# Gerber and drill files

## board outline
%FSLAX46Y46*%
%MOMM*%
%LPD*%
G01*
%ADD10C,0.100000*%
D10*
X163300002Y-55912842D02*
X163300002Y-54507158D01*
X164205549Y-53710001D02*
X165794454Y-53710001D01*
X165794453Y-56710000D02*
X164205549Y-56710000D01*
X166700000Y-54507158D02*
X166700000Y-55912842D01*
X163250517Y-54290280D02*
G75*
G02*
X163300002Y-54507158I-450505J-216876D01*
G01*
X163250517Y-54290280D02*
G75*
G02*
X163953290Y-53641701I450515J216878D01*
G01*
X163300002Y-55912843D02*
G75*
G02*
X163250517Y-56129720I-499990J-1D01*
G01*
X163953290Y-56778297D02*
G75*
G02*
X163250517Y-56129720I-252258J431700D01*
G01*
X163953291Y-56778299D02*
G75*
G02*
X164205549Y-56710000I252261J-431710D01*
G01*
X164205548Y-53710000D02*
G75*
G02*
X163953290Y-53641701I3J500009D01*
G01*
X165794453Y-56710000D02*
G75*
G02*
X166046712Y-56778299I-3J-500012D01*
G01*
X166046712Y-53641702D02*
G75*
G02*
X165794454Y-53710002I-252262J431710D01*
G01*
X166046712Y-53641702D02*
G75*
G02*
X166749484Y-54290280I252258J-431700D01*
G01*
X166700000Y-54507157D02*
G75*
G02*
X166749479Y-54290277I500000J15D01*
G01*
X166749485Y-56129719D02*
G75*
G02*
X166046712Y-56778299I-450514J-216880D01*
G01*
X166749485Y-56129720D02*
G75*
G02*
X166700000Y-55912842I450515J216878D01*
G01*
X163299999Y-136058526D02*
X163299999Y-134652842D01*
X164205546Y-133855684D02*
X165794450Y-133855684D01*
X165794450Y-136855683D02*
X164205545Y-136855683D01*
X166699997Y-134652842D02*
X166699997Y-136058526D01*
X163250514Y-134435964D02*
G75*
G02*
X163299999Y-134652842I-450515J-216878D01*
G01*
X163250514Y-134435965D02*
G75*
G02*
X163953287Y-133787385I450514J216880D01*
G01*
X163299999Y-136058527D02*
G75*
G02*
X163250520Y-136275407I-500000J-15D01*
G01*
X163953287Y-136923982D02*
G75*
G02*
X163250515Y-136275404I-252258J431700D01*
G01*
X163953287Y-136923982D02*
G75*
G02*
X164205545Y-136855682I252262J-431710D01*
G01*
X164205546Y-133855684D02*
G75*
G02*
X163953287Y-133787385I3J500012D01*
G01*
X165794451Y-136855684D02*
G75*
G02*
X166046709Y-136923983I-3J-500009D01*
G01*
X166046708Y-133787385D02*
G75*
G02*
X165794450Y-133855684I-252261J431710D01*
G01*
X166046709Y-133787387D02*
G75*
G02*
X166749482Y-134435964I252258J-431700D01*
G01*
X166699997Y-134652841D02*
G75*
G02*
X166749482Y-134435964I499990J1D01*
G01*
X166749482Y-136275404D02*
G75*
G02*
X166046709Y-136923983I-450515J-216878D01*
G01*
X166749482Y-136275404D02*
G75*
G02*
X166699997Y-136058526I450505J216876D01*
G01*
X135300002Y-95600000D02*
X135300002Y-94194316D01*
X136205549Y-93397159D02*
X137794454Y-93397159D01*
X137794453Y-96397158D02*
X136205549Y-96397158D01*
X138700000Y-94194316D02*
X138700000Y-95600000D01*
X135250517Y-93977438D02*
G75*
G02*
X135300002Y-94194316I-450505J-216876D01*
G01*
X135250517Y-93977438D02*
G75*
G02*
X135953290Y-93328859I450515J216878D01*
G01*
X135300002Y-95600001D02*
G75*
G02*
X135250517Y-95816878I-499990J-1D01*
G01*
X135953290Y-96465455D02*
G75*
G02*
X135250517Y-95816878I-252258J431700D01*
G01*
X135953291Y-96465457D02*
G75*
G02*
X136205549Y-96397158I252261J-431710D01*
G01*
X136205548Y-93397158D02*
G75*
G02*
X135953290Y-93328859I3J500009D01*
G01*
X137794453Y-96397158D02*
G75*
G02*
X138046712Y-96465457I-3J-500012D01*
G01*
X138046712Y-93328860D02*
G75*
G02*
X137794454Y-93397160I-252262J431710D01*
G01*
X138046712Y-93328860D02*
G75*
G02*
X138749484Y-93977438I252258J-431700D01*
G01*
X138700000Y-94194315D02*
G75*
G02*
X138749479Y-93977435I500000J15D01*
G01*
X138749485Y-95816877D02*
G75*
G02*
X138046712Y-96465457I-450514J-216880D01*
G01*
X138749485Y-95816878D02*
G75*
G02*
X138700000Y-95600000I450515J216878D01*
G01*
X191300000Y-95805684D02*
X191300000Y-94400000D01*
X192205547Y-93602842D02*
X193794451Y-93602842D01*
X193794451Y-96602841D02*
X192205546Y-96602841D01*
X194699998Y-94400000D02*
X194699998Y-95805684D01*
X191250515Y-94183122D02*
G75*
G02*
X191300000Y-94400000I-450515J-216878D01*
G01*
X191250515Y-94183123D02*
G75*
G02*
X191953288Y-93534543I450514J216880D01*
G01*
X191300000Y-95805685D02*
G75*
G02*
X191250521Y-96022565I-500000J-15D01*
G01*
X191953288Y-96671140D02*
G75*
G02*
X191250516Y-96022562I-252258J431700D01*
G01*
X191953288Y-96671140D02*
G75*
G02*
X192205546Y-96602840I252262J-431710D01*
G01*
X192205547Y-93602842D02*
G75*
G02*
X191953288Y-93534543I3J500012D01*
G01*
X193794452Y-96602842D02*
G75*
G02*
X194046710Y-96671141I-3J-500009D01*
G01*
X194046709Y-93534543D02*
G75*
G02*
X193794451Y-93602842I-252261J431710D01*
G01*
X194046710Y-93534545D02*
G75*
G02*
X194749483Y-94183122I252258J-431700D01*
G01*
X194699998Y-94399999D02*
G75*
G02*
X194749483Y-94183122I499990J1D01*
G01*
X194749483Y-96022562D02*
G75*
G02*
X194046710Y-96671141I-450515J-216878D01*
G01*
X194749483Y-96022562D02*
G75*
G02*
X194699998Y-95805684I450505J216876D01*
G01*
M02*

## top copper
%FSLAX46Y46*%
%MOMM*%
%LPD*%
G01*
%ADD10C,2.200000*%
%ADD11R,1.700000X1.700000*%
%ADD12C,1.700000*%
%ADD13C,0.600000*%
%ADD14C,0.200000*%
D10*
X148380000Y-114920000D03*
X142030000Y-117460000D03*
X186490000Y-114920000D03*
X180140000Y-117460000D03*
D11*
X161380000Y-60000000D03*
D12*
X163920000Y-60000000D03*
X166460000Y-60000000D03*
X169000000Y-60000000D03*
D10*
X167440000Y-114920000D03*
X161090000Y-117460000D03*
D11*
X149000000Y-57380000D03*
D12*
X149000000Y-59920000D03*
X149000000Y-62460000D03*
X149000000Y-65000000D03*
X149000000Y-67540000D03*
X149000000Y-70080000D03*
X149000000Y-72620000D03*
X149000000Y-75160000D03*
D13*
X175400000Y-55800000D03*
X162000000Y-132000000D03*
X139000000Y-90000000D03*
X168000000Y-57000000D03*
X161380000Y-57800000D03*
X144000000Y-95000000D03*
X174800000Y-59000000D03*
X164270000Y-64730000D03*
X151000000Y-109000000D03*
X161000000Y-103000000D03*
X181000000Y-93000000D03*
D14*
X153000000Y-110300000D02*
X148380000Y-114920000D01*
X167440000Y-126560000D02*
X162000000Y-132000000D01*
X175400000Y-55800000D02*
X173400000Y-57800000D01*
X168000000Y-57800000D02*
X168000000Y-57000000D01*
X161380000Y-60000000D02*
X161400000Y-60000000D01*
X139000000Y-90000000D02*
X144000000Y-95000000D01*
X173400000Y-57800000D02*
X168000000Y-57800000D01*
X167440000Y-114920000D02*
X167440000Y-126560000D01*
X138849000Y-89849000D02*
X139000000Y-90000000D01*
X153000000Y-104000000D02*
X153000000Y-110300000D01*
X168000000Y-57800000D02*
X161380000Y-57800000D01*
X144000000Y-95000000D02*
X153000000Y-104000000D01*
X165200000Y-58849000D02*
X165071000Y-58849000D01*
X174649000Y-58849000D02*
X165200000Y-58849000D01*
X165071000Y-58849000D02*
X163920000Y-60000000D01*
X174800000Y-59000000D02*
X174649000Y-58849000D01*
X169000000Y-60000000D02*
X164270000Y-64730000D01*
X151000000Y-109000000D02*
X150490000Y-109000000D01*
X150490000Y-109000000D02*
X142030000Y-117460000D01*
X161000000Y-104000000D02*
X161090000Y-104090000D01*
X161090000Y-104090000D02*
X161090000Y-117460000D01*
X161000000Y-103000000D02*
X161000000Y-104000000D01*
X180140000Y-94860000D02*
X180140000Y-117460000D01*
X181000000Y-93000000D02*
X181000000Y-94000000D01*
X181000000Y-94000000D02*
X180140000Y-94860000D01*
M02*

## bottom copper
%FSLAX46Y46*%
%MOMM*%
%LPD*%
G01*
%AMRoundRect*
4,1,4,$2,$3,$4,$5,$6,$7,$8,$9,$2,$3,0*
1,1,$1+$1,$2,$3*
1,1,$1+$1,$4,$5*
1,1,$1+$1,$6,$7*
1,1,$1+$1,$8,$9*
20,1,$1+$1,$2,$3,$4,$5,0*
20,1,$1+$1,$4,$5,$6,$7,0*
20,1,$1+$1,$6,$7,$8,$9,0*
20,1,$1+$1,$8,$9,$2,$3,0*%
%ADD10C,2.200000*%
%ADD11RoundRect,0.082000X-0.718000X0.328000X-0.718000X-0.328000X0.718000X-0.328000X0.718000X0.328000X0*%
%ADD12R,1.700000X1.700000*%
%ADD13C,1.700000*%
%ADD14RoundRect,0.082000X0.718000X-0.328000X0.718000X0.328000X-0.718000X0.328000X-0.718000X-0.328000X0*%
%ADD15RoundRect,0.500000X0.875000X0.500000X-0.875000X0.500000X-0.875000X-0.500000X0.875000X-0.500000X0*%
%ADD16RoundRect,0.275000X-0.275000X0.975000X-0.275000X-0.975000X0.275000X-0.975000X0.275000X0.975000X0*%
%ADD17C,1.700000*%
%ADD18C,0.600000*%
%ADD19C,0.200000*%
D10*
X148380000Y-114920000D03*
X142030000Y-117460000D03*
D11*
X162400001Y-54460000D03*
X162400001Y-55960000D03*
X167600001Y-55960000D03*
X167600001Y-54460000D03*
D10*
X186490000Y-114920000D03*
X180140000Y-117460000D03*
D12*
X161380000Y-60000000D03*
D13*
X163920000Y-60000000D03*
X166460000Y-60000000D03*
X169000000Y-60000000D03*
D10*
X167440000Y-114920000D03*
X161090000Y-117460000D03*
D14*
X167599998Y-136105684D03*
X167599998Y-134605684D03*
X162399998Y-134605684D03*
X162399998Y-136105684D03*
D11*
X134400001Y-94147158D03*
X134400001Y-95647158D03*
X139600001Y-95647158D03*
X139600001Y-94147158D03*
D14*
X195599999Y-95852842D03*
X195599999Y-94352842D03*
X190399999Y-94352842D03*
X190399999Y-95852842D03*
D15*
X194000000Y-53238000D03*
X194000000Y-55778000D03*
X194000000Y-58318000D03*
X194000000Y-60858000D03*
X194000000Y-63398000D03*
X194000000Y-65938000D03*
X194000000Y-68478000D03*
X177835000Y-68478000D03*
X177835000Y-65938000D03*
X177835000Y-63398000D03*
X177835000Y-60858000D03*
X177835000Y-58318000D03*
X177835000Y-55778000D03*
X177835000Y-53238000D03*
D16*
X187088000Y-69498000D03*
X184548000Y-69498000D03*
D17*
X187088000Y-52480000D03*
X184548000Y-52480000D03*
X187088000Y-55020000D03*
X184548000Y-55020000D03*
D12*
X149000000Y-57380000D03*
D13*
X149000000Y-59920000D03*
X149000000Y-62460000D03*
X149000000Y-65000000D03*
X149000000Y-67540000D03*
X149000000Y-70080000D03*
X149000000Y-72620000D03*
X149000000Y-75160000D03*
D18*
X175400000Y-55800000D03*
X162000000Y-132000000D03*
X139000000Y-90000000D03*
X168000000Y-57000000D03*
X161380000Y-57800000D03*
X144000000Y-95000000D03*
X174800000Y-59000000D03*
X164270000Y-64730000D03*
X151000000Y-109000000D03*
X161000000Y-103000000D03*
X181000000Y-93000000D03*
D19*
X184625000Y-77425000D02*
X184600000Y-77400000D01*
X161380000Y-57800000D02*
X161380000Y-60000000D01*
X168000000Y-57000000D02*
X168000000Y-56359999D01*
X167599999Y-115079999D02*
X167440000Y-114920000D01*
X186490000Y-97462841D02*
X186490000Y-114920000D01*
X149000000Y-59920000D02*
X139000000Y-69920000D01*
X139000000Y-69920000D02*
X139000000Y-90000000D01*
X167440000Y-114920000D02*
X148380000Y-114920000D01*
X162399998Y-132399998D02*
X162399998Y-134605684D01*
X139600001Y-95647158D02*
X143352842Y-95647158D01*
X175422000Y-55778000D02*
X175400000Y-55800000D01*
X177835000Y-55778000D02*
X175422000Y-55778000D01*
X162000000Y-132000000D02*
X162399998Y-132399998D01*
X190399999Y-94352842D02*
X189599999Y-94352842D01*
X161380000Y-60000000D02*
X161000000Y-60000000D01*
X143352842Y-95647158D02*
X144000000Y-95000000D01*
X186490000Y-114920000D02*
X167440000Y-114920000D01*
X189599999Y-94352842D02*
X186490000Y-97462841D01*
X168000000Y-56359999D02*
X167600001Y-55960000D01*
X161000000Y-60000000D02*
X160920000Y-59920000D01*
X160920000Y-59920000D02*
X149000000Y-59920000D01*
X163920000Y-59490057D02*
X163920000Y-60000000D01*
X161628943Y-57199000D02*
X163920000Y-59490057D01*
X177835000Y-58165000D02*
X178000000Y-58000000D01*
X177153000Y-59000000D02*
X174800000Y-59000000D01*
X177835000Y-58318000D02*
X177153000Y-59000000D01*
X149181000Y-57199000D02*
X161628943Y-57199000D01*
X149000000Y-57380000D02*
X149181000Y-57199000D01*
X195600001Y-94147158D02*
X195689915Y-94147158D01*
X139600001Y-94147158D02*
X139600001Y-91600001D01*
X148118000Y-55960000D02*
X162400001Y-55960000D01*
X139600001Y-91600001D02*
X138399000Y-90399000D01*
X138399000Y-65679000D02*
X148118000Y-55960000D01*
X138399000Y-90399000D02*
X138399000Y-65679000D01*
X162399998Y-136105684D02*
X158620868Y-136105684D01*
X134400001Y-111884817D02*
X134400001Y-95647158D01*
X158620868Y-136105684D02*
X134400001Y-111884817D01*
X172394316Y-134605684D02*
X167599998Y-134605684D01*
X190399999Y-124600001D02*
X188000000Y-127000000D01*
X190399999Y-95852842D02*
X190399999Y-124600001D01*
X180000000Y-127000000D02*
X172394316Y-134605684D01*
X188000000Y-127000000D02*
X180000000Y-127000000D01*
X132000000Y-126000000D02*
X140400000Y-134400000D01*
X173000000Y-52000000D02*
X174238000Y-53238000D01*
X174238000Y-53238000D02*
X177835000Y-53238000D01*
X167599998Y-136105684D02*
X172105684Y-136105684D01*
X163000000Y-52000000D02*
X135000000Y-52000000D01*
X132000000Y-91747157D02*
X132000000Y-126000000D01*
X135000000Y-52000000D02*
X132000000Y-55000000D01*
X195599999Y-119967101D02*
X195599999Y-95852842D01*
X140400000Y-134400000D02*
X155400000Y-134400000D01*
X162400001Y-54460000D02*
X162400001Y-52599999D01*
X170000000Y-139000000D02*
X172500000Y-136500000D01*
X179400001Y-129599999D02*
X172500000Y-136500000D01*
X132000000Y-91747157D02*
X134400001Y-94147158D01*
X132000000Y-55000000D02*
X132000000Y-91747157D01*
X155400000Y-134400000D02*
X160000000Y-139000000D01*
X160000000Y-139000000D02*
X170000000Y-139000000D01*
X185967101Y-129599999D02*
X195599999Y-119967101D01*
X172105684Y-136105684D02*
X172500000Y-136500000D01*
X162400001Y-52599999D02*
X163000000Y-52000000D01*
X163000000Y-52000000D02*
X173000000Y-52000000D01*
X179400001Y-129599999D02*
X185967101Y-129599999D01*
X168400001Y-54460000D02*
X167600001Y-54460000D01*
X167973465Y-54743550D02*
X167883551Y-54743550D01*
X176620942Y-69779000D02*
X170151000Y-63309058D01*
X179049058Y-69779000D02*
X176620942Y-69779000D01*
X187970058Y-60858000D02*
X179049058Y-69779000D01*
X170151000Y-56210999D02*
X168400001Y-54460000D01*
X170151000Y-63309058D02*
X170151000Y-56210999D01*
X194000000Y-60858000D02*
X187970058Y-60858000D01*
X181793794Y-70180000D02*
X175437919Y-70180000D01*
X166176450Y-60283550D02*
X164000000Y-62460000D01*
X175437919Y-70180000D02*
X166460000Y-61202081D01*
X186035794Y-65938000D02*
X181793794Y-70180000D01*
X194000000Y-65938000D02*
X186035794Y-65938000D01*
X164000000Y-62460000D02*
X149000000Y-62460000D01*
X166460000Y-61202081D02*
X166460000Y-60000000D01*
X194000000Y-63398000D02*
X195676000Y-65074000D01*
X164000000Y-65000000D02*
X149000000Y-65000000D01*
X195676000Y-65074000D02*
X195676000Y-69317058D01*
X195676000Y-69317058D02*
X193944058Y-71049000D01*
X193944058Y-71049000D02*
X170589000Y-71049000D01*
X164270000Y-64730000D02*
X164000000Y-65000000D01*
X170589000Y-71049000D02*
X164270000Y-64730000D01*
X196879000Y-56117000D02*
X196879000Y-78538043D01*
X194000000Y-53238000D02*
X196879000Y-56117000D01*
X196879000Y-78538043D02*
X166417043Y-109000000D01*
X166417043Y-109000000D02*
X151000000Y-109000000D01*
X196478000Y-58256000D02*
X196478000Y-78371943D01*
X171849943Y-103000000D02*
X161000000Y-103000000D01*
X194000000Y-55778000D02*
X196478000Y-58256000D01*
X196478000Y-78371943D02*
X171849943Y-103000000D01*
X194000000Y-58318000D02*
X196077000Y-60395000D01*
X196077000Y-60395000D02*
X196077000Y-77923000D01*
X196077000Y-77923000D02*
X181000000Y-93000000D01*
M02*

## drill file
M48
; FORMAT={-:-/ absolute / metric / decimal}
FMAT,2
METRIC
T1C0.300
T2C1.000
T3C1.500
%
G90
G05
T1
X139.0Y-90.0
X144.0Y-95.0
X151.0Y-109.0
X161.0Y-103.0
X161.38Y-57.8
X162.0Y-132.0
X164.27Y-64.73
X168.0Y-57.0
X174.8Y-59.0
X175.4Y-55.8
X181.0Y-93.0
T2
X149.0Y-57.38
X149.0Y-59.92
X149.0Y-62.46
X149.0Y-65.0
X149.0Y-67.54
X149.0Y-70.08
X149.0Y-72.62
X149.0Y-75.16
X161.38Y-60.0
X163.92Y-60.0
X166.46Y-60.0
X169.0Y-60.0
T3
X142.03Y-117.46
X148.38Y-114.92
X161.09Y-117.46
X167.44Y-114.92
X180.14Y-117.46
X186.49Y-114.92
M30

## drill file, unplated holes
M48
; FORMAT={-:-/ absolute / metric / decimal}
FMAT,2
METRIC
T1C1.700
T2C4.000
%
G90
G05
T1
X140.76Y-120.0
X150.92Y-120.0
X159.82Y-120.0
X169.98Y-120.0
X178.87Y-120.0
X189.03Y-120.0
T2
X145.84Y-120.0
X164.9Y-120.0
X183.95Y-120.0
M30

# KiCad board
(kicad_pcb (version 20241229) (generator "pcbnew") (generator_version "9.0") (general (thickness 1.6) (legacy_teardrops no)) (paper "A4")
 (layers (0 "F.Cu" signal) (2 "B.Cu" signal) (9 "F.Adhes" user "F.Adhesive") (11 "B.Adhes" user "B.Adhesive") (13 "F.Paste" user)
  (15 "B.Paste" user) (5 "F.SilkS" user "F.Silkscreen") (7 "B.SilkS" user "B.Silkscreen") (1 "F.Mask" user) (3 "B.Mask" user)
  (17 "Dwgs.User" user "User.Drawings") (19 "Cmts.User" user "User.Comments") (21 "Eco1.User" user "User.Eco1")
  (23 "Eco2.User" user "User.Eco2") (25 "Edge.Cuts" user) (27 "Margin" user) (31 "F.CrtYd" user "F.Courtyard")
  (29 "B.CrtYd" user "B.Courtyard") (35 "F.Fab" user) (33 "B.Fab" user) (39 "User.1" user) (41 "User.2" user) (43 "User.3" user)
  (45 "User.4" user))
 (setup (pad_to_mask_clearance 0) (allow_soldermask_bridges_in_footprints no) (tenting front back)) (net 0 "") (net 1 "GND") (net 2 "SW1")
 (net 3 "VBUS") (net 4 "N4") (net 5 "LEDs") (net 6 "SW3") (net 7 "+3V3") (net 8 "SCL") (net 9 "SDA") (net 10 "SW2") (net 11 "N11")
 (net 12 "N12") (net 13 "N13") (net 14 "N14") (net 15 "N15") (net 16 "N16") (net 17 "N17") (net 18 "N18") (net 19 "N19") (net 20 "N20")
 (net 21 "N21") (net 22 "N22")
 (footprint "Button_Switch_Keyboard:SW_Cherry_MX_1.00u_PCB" (layer "F.Cu") (at 148.38 114.92)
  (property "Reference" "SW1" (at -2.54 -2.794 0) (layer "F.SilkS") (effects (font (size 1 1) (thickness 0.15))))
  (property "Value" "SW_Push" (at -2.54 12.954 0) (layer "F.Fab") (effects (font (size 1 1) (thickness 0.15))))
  (pad "" np_thru_hole circle (at -7.62 5.08) (size 1.7 1.7) (drill 1.7) (layers "*.Cu" "*.Mask"))
  (pad "" np_thru_hole circle (at -2.54 5.08) (size 4 4) (drill 4) (layers "*.Cu" "*.Mask"))
  (pad "" np_thru_hole circle (at 2.54 5.08) (size 1.7 1.7) (drill 1.7) (layers "*.Cu" "*.Mask"))
  (pad "1" thru_hole circle (at 0 0) (size 2.2 2.2) (drill 1.5) (layers "*.Cu" "*.Mask") (remove_unused_layers no) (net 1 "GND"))
  (pad "2" thru_hole circle (at -6.35 2.54) (size 2.2 2.2) (drill 1.5) (layers "*.Cu" "*.Mask") (remove_unused_layers no) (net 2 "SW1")))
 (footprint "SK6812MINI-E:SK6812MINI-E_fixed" (layer "F.Cu") (at 165 55.312842)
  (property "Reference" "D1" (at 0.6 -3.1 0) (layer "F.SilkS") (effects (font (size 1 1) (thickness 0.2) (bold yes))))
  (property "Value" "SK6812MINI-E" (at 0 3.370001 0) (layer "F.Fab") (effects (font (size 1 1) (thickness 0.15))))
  (fp_line (start -1.699998 0.6) (end -1.699998 -0.805684) (stroke (width 0.1) (type solid)) (layer "Edge.Cuts"))
  (fp_line (start -0.794451 -1.602841) (end 0.794454 -1.602841) (stroke (width 0.1) (type solid)) (layer "Edge.Cuts"))
  (fp_line (start 0.794453 1.397158) (end -0.794451 1.397158) (stroke (width 0.1) (type solid)) (layer "Edge.Cuts"))
  (fp_line (start 1.7 -0.805684) (end 1.7 0.6) (stroke (width 0.1) (type solid)) (layer "Edge.Cuts"))
  (fp_arc (start -1.749483 -1.022562) (mid -1.712526 -0.91691) (end -1.699998 -0.805684) (stroke (width 0.1) (type solid))
   (layer "Edge.Cuts"))
  (fp_arc (start -1.749483 -1.022562) (mid -1.63807 -1.606877) (end -1.04671 -1.671141) (stroke (width 0.1) (type solid))
   (layer "Edge.Cuts"))
  (fp_arc (start -1.699998 0.600001) (mid -1.712526 0.711226) (end -1.749483 0.816878) (stroke (width 0.1) (type solid)) (layer "Edge.Cuts"))
  (fp_arc (start -1.04671 1.465455) (mid -1.638069 1.401192) (end -1.749483 0.816878) (stroke (width 0.1) (type solid)) (layer "Edge.Cuts"))
  (fp_arc (start -1.046709 1.465457) (mid -0.925121 1.414535) (end -0.794451 1.397158) (stroke (width 0.1) (type solid)) (layer "Edge.Cuts"))
  (fp_arc (start -0.794452 -1.602842) (mid -0.925122 -1.620219) (end -1.04671 -1.671141) (stroke (width 0.1) (type solid))
   (layer "Edge.Cuts"))
  (fp_arc (start 0.794453 1.397158) (mid 0.925124 1.414535) (end 1.046712 1.465457) (stroke (width 0.1) (type solid)) (layer "Edge.Cuts"))
  (fp_arc (start 1.046712 -1.67114) (mid 0.925124 -1.620218) (end 0.794454 -1.602841) (stroke (width 0.1) (type solid)) (layer "Edge.Cuts"))
  (fp_arc (start 1.046712 -1.67114) (mid 1.638072 -1.606876) (end 1.749485 -1.022562) (stroke (width 0.1) (type solid)) (layer "Edge.Cuts"))
  (fp_arc (start 1.7 -0.805685) (mid 1.712528 -0.91691) (end 1.749485 -1.022562) (stroke (width 0.1) (type solid)) (layer "Edge.Cuts"))
  (fp_arc (start 1.749485 0.816877) (mid 1.638073 1.401193) (end 1.046712 1.465457) (stroke (width 0.1) (type solid)) (layer "Edge.Cuts"))
  (fp_arc (start 1.749485 0.816878) (mid 1.712528 0.711226) (end 1.7 0.6) (stroke (width 0.1) (type solid)) (layer "Edge.Cuts"))
  (pad "1" smd roundrect (at -2.599999 -0.852842 270) (size 0.82 1.6) (layers "B.Cu" "B.Mask" "B.Paste") (roundrect_rratio 0.1)
   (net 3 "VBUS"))
  (pad "2" smd roundrect (at -2.599999 0.647158 270) (size 0.82 1.6) (layers "B.Cu" "B.Mask" "B.Paste") (roundrect_rratio 0.1) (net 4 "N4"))
  (pad "3" smd roundrect (at 2.600001 0.647158 270) (size 0.82 1.6) (layers "B.Cu" "B.Mask" "B.Paste") (roundrect_rratio 0.1) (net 1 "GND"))
  (pad "4" smd roundrect (at 2.600001 -0.852842 270) (size 0.82 1.6) (layers "B.Cu" "B.Mask" "B.Paste") (roundrect_rratio 0.1)
   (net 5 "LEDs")))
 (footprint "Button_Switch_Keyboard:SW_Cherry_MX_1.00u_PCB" (layer "F.Cu") (at 186.49 114.92)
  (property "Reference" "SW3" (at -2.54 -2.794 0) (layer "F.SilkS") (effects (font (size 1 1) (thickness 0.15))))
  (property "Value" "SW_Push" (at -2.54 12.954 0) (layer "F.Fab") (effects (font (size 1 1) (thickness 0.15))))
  (pad "" np_thru_hole circle (at -7.62 5.08) (size 1.7 1.7) (drill 1.7) (layers "*.Cu" "*.Mask"))
  (pad "" np_thru_hole circle (at -2.54 5.08) (size 4 4) (drill 4) (layers "*.Cu" "*.Mask"))
  (pad "" np_thru_hole circle (at 2.54 5.08) (size 1.7 1.7) (drill 1.7) (layers "*.Cu" "*.Mask"))
  (pad "1" thru_hole circle (at 0 0) (size 2.2 2.2) (drill 1.5) (layers "*.Cu" "*.Mask") (remove_unused_layers no) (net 1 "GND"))
  (pad "2" thru_hole circle (at -6.35 2.54) (size 2.2 2.2) (drill 1.5) (layers "*.Cu" "*.Mask") (remove_unused_layers no) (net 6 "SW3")))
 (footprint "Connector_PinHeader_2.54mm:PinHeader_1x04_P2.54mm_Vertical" (layer "F.Cu") (at 161.38 60 90)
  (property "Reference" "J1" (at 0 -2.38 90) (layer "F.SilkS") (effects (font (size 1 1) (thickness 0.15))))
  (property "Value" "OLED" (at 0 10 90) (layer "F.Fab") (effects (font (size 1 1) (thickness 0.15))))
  (pad "1" thru_hole rect (at 0 0 90) (size 1.7 1.7) (drill 1) (layers "*.Cu" "*.Mask") (remove_unused_layers no) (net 1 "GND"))
  (pad "2" thru_hole circle (at 0 2.54 90) (size 1.7 1.7) (drill 1) (layers "*.Cu" "*.Mask") (remove_unused_layers no) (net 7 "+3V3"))
  (pad "3" thru_hole circle (at 0 5.08 90) (size 1.7 1.7) (drill 1) (layers "*.Cu" "*.Mask") (remove_unused_layers no) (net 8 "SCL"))
  (pad "4" thru_hole circle (at 0 7.62 90) (size 1.7 1.7) (drill 1) (layers "*.Cu" "*.Mask") (remove_unused_layers no) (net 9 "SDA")))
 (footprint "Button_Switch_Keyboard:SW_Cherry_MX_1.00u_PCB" (layer "F.Cu") (at 167.44 114.92)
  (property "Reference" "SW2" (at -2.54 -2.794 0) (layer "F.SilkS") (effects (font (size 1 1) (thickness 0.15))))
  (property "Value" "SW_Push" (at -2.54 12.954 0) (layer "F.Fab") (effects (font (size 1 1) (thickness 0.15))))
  (pad "" np_thru_hole circle (at -7.62 5.08) (size 1.7 1.7) (drill 1.7) (layers "*.Cu" "*.Mask"))
  (pad "" np_thru_hole circle (at -2.54 5.08) (size 4 4) (drill 4) (layers "*.Cu" "*.Mask"))
  (pad "" np_thru_hole circle (at 2.54 5.08) (size 1.7 1.7) (drill 1.7) (layers "*.Cu" "*.Mask"))
  (pad "1" thru_hole circle (at 0 0) (size 2.2 2.2) (drill 1.5) (layers "*.Cu" "*.Mask") (remove_unused_layers no) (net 1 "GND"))
  (pad "2" thru_hole circle (at -6.35 2.54) (size 2.2 2.2) (drill 1.5) (layers "*.Cu" "*.Mask") (remove_unused_layers no) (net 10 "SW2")))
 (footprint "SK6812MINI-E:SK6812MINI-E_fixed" (layer "F.Cu") (at 164.999999 135.252842 180)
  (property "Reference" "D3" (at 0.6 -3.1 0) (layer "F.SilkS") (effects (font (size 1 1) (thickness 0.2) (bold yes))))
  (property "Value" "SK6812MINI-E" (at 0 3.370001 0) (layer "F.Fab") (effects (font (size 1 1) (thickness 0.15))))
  (fp_line (start 1.7 -0.805684) (end 1.7 0.6) (stroke (width 0.1) (type solid)) (layer "Edge.Cuts"))
  (fp_line (start 0.794453 1.397158) (end -0.794451 1.397158) (stroke (width 0.1) (type solid)) (layer "Edge.Cuts"))
  (fp_line (start -0.794451 -1.602841) (end 0.794454 -1.602841) (stroke (width 0.1) (type solid)) (layer "Edge.Cuts"))
  (fp_line (start -1.699998 0.6) (end -1.699998 -0.805684) (stroke (width 0.1) (type solid)) (layer "Edge.Cuts"))
  (fp_arc (start 1.749485 0.816878) (mid 1.712528 0.711226) (end 1.7 0.6) (stroke (width 0.1) (type solid)) (layer "Edge.Cuts"))
  (fp_arc (start 1.749485 0.816877) (mid 1.638073 1.401193) (end 1.046712 1.465457) (stroke (width 0.1) (type solid)) (layer "Edge.Cuts"))
  (fp_arc (start 1.7 -0.805685) (mid 1.712528 -0.91691) (end 1.749485 -1.022562) (stroke (width 0.1) (type solid)) (layer "Edge.Cuts"))
  (fp_arc (start 1.046712 -1.67114) (mid 1.638072 -1.606876) (end 1.749485 -1.022562) (stroke (width 0.1) (type solid)) (layer "Edge.Cuts"))
  (fp_arc (start 1.046712 -1.67114) (mid 0.925124 -1.620218) (end 0.794454 -1.602841) (stroke (width 0.1) (type solid)) (layer "Edge.Cuts"))
  (fp_arc (start 0.794453 1.397158) (mid 0.925124 1.414535) (end 1.046712 1.465457) (stroke (width 0.1) (type solid)) (layer "Edge.Cuts"))
  (fp_arc (start -0.794452 -1.602842) (mid -0.925122 -1.620219) (end -1.04671 -1.671141) (stroke (width 0.1) (type solid))
   (layer "Edge.Cuts"))
  (fp_arc (start -1.046709 1.465457) (mid -0.925121 1.414535) (end -0.794451 1.397158) (stroke (width 0.1) (type solid)) (layer "Edge.Cuts"))
  (fp_arc (start -1.04671 1.465455) (mid -1.638069 1.401192) (end -1.749483 0.816878) (stroke (width 0.1) (type solid)) (layer "Edge.Cuts"))
  (fp_arc (start -1.699998 0.600001) (mid -1.712526 0.711226) (end -1.749483 0.816878) (stroke (width 0.1) (type solid)) (layer "Edge.Cuts"))
  (fp_arc (start -1.749483 -1.022562) (mid -1.63807 -1.606877) (end -1.04671 -1.671141) (stroke (width 0.1) (type solid))
   (layer "Edge.Cuts"))
  (fp_arc (start -1.749483 -1.022562) (mid -1.712526 -0.91691) (end -1.699998 -0.805684) (stroke (width 0.1) (type solid))
   (layer "Edge.Cuts"))
  (pad "1" smd roundrect (at -2.599999 -0.852842 90) (size 0.82 1.6) (layers "B.Cu" "B.Mask" "B.Paste") (roundrect_rratio 0.1)
   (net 3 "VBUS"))
  (pad "2" smd roundrect (at -2.599999 0.647158 90) (size 0.82 1.6) (layers "B.Cu" "B.Mask" "B.Paste") (roundrect_rratio 0.1) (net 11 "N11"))
  (pad "3" smd roundrect (at 2.600001 0.647158 90) (size 0.82 1.6) (layers "B.Cu" "B.Mask" "B.Paste") (roundrect_rratio 0.1) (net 1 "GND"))
  (pad "4" smd roundrect (at 2.600001 -0.852842 90) (size 0.82 1.6) (layers "B.Cu" "B.Mask" "B.Paste") (roundrect_rratio 0.1) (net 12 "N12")))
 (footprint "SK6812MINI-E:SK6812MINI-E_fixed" (layer "F.Cu") (at 137 95)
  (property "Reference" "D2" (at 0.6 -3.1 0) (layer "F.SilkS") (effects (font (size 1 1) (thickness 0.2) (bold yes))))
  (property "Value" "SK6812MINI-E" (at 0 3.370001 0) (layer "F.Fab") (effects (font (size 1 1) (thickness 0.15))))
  (fp_line (start -1.699998 0.6) (end -1.699998 -0.805684) (stroke (width 0.1) (type solid)) (layer "Edge.Cuts"))
  (fp_line (start -0.794451 -1.602841) (end 0.794454 -1.602841) (stroke (width 0.1) (type solid)) (layer "Edge.Cuts"))
  (fp_line (start 0.794453 1.397158) (end -0.794451 1.397158) (stroke (width 0.1) (type solid)) (layer "Edge.Cuts"))
  (fp_line (start 1.7 -0.805684) (end 1.7 0.6) (stroke (width 0.1) (type solid)) (layer "Edge.Cuts"))
  (fp_arc (start -1.749483 -1.022562) (mid -1.712526 -0.91691) (end -1.699998 -0.805684) (stroke (width 0.1) (type solid))
   (layer "Edge.Cuts"))
  (fp_arc (start -1.749483 -1.022562) (mid -1.63807 -1.606877) (end -1.04671 -1.671141) (stroke (width 0.1) (type solid))
   (layer "Edge.Cuts"))
  (fp_arc (start -1.699998 0.600001) (mid -1.712526 0.711226) (end -1.749483 0.816878) (stroke (width 0.1) (type solid)) (layer "Edge.Cuts"))
  (fp_arc (start -1.04671 1.465455) (mid -1.638069 1.401192) (end -1.749483 0.816878) (stroke (width 0.1) (type solid)) (layer "Edge.Cuts"))
  (fp_arc (start -1.046709 1.465457) (mid -0.925121 1.414535) (end -0.794451 1.397158) (stroke (width 0.1) (type solid)) (layer "Edge.Cuts"))
  (fp_arc (start -0.794452 -1.602842) (mid -0.925122 -1.620219) (end -1.04671 -1.671141) (stroke (width 0.1) (type solid))
   (layer "Edge.Cuts"))
  (fp_arc (start 0.794453 1.397158) (mid 0.925124 1.414535) (end 1.046712 1.465457) (stroke (width 0.1) (type solid)) (layer "Edge.Cuts"))
  (fp_arc (start 1.046712 -1.67114) (mid 0.925124 -1.620218) (end 0.794454 -1.602841) (stroke (width 0.1) (type solid)) (layer "Edge.Cuts"))
  (fp_arc (start 1.046712 -1.67114) (mid 1.638072 -1.606876) (end 1.749485 -1.022562) (stroke (width 0.1) (type solid)) (layer "Edge.Cuts"))
  (fp_arc (start 1.7 -0.805685) (mid 1.712528 -0.91691) (end 1.749485 -1.022562) (stroke (width 0.1) (type solid)) (layer "Edge.Cuts"))
  (fp_arc (start 1.749485 0.816877) (mid 1.638073 1.401193) (end 1.046712 1.465457) (stroke (width 0.1) (type solid)) (layer "Edge.Cuts"))
  (fp_arc (start 1.749485 0.816878) (mid 1.712528 0.711226) (end 1.7 0.6) (stroke (width 0.1) (type solid)) (layer "Edge.Cuts"))
  (pad "1" smd roundrect (at -2.599999 -0.852842 270) (size 0.82 1.6) (layers "B.Cu" "B.Mask" "B.Paste") (roundrect_rratio 0.1)
   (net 3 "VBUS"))
  (pad "2" smd roundrect (at -2.599999 0.647158 270) (size 0.82 1.6) (layers "B.Cu" "B.Mask" "B.Paste") (roundrect_rratio 0.1)
   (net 12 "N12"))
  (pad "3" smd roundrect (at 2.600001 0.647158 270) (size 0.82 1.6) (layers "B.Cu" "B.Mask" "B.Paste") (roundrect_rratio 0.1) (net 1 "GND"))
  (pad "4" smd roundrect (at 2.600001 -0.852842 270) (size 0.82 1.6) (layers "B.Cu" "B.Mask" "B.Paste") (roundrect_rratio 0.1) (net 4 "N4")))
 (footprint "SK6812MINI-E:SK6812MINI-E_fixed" (layer "F.Cu") (at 193 95 180)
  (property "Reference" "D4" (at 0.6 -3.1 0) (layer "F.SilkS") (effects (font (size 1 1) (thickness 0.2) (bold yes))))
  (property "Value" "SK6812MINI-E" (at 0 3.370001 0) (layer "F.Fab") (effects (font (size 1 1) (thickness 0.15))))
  (fp_line (start 1.7 -0.805684) (end 1.7 0.6) (stroke (width 0.1) (type solid)) (layer "Edge.Cuts"))
  (fp_line (start 0.794453 1.397158) (end -0.794451 1.397158) (stroke (width 0.1) (type solid)) (layer "Edge.Cuts"))
  (fp_line (start -0.794451 -1.602841) (end 0.794454 -1.602841) (stroke (width 0.1) (type solid)) (layer "Edge.Cuts"))
  (fp_line (start -1.699998 0.6) (end -1.699998 -0.805684) (stroke (width 0.1) (type solid)) (layer "Edge.Cuts"))
  (fp_arc (start 1.749485 0.816878) (mid 1.712528 0.711226) (end 1.7 0.6) (stroke (width 0.1) (type solid)) (layer "Edge.Cuts"))
  (fp_arc (start 1.749485 0.816877) (mid 1.638073 1.401193) (end 1.046712 1.465457) (stroke (width 0.1) (type solid)) (layer "Edge.Cuts"))
  (fp_arc (start 1.7 -0.805685) (mid 1.712528 -0.91691) (end 1.749485 -1.022562) (stroke (width 0.1) (type solid)) (layer "Edge.Cuts"))
  (fp_arc (start 1.046712 -1.67114) (mid 1.638072 -1.606876) (end 1.749485 -1.022562) (stroke (width 0.1) (type solid)) (layer "Edge.Cuts"))
  (fp_arc (start 1.046712 -1.67114) (mid 0.925124 -1.620218) (end 0.794454 -1.602841) (stroke (width 0.1) (type solid)) (layer "Edge.Cuts"))
  (fp_arc (start 0.794453 1.397158) (mid 0.925124 1.414535) (end 1.046712 1.465457) (stroke (width 0.1) (type solid)) (layer "Edge.Cuts"))
  (fp_arc (start -0.794452 -1.602842) (mid -0.925122 -1.620219) (end -1.04671 -1.671141) (stroke (width 0.1) (type solid))
   (layer "Edge.Cuts"))
  (fp_arc (start -1.046709 1.465457) (mid -0.925121 1.414535) (end -0.794451 1.397158) (stroke (width 0.1) (type solid)) (layer "Edge.Cuts"))
  (fp_arc (start -1.04671 1.465455) (mid -1.638069 1.401192) (end -1.749483 0.816878) (stroke (width 0.1) (type solid)) (layer "Edge.Cuts"))
  (fp_arc (start -1.699998 0.600001) (mid -1.712526 0.711226) (end -1.749483 0.816878) (stroke (width 0.1) (type solid)) (layer "Edge.Cuts"))
  (fp_arc (start -1.749483 -1.022562) (mid -1.63807 -1.606877) (end -1.04671 -1.671141) (stroke (width 0.1) (type solid))
   (layer "Edge.Cuts"))
  (fp_arc (start -1.749483 -1.022562) (mid -1.712526 -0.91691) (end -1.699998 -0.805684) (stroke (width 0.1) (type solid))
   (layer "Edge.Cuts"))
  (pad "1" smd roundrect (at -2.599999 -0.852842 90) (size 0.82 1.6) (layers "B.Cu" "B.Mask" "B.Paste") (roundrect_rratio 0.1)
   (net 3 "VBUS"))
  (pad "2" smd roundrect (at -2.599999 0.647158 90) (size 0.82 1.6) (layers "B.Cu" "B.Mask" "B.Paste") (roundrect_rratio 0.1) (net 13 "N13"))
  (pad "3" smd roundrect (at 2.600001 0.647158 90) (size 0.82 1.6) (layers "B.Cu" "B.Mask" "B.Paste") (roundrect_rratio 0.1) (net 1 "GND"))
  (pad "4" smd roundrect (at 2.600001 -0.852842 90) (size 0.82 1.6) (layers "B.Cu" "B.Mask" "B.Paste") (roundrect_rratio 0.1) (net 11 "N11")))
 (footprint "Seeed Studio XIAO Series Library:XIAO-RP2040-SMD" (layer "B.Cu") (at 186 60.858 180)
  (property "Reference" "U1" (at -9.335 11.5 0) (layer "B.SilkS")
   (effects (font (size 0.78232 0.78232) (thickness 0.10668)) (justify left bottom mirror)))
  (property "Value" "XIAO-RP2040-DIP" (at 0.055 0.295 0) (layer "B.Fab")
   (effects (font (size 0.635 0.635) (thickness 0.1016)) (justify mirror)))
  (pad "1" smd roundrect (at -8 7.62 180) (size 2.75 2) (layers "B.Cu" "B.Mask" "B.Paste") (roundrect_rratio 0.25) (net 2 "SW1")
   (solder_mask_margin 0.0508) (thermal_bridge_angle 45))
  (pad "2" smd roundrect (at -8 5.08 180) (size 2.75 2) (layers "B.Cu" "B.Mask" "B.Paste") (roundrect_rratio 0.25) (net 10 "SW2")
   (solder_mask_margin 0.0508) (thermal_bridge_angle 45))
  (pad "3" smd roundrect (at -8 2.54 180) (size 2.75 2) (layers "B.Cu" "B.Mask" "B.Paste") (roundrect_rratio 0.25) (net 6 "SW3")
   (solder_mask_margin 0.0508) (thermal_bridge_angle 45))
  (pad "4" smd roundrect (at -8 0 180) (size 2.75 2) (layers "B.Cu" "B.Mask" "B.Paste") (roundrect_rratio 0.25) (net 5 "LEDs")
   (solder_mask_margin 0.0508) (thermal_bridge_angle 45))
  (pad "5" smd roundrect (at -8 -2.54 180) (size 2.75 2) (layers "B.Cu" "B.Mask" "B.Paste") (roundrect_rratio 0.25) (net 9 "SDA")
   (solder_mask_margin 0.0508) (thermal_bridge_angle 45))
  (pad "6" smd roundrect (at -8 -5.08 180) (size 2.75 2) (layers "B.Cu" "B.Mask" "B.Paste") (roundrect_rratio 0.25) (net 8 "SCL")
   (solder_mask_margin 0.0508) (thermal_bridge_angle 45))
  (pad "7" smd roundrect (at -8 -7.62 180) (size 2.75 2) (layers "B.Cu" "B.Mask" "B.Paste") (roundrect_rratio 0.25) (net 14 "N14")
   (solder_mask_margin 0.0508) (thermal_bridge_angle 45))
  (pad "8" smd roundrect (at 8.165 -7.62 180) (size 2.75 2) (layers "B.Cu" "B.Mask" "B.Paste") (roundrect_rratio 0.25) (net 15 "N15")
   (solder_mask_margin 0.0508) (thermal_bridge_angle 45))
  (pad "9" smd roundrect (at 8.165 -5.08 180) (size 2.75 2) (layers "B.Cu" "B.Mask" "B.Paste") (roundrect_rratio 0.25) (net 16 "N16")
   (solder_mask_margin 0.0508) (thermal_bridge_angle 45))
  (pad "10" smd roundrect (at 8.165 -2.54 180) (size 2.75 2) (layers "B.Cu" "B.Mask" "B.Paste") (roundrect_rratio 0.25) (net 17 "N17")
   (solder_mask_margin 0.0508) (thermal_bridge_angle 45))
  (pad "11" smd roundrect (at 8.165 0 180) (size 2.75 2) (layers "B.Cu" "B.Mask" "B.Paste") (roundrect_rratio 0.25) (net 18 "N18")
   (solder_mask_margin 0.0508) (thermal_bridge_angle 45))
  (pad "12" smd roundrect (at 8.165 2.54 180) (size 2.75 2) (layers "B.Cu" "B.Mask" "B.Paste") (roundrect_rratio 0.25) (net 7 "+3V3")
   (solder_mask_margin 0.0508) (thermal_bridge_angle 45))
  (pad "13" smd roundrect (at 8.165 5.08 180) (size 2.75 2) (layers "B.Cu" "B.Mask" "B.Paste") (roundrect_rratio 0.25) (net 1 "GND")
   (solder_mask_margin 0.0508) (thermal_bridge_angle 45))
  (pad "14" smd roundrect (at 8.165 7.62 180) (size 2.75 2) (layers "B.Cu" "B.Mask" "B.Paste") (roundrect_rratio 0.25) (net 3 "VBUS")
   (solder_mask_margin 0.0508) (thermal_bridge_angle 45))
  (pad "15" smd roundrect (at -1.088 -8.64 270) (size 2.5 1.1) (layers "B.Cu" "B.Mask" "B.Paste") (roundrect_rratio 0.25)
   (thermal_bridge_angle 45))
  (pad "16" smd roundrect (at 1.452 -8.64 270) (size 2.5 1.1) (layers "B.Cu" "B.Mask" "B.Paste") (roundrect_rratio 0.25)
   (thermal_bridge_angle 45))
  (pad "17" smd circle (at -1.088 8.378 180) (size 1.7 1.7) (layers "B.Cu" "B.Mask" "B.Paste"))
  (pad "18" smd circle (at 1.452 8.378 180) (size 1.7 1.7) (layers "B.Cu" "B.Mask" "B.Paste"))
  (pad "19" smd circle (at -1.088 5.838 180) (size 1.7 1.7) (layers "B.Cu" "B.Mask" "B.Paste"))
  (pad "20" smd circle (at 1.452 5.838 180) (size 1.7 1.7) (layers "B.Cu" "B.Mask" "B.Paste")))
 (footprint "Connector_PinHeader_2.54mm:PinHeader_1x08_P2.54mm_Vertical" (layer "B.Cu") (at 149 57.38 180)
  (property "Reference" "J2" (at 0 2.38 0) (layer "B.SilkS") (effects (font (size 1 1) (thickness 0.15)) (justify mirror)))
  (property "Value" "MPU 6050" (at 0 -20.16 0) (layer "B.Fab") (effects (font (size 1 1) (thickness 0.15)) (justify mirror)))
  (pad "1" thru_hole rect (at 0 0 180) (size 1.7 1.7) (drill 1) (layers "*.Cu" "*.Mask") (remove_unused_layers no) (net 7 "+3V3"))
  (pad "2" thru_hole circle (at 0 -2.54 180) (size 1.7 1.7) (drill 1) (layers "*.Cu" "*.Mask") (remove_unused_layers no) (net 1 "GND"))
  (pad "3" thru_hole circle (at 0 -5.08 180) (size 1.7 1.7) (drill 1) (layers "*.Cu" "*.Mask") (remove_unused_layers no) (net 8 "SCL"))
  (pad "4" thru_hole circle (at 0 -7.62 180) (size 1.7 1.7) (drill 1) (layers "*.Cu" "*.Mask") (remove_unused_layers no) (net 9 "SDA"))
  (pad "5" thru_hole circle (at 0 -10.16 180) (size 1.7 1.7) (drill 1) (layers "*.Cu" "*.Mask") (remove_unused_layers no) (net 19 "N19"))
  (pad "6" thru_hole circle (at 0 -12.7 180) (size 1.7 1.7) (drill 1) (layers "*.Cu" "*.Mask") (remove_unused_layers no) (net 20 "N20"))
  (pad "7" thru_hole circle (at 0 -15.24 180) (size 1.7 1.7) (drill 1) (layers "*.Cu" "*.Mask") (remove_unused_layers no) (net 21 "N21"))
  (pad "8" thru_hole circle (at 0 -17.78 180) (size 1.7 1.7) (drill 1) (layers "*.Cu" "*.Mask") (remove_unused_layers no) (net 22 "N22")))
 (segment (start 184.625 77.425) (end 184.6 77.4) (width 0.2) (layer "B.Cu") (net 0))
 (segment (start 153 110.3) (end 148.38 114.92) (width 0.2) (layer "F.Cu") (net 1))
 (segment (start 167.44 126.56) (end 162 132) (width 0.2) (layer "F.Cu") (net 1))
 (segment (start 175.4 55.8) (end 173.4 57.8) (width 0.2) (layer "F.Cu") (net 1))
 (segment (start 168 57.8) (end 168 57) (width 0.2) (layer "F.Cu") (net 1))
 (segment (start 161.38 60) (end 161.4 60) (width 0.2) (layer "F.Cu") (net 1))
 (segment (start 139 90) (end 144 95) (width 0.2) (layer "F.Cu") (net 1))
 (segment (start 173.4 57.8) (end 168 57.8) (width 0.2) (layer "F.Cu") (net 1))
 (segment (start 167.44 114.92) (end 167.44 126.56) (width 0.2) (layer "F.Cu") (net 1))
 (segment (start 138.849 89.849) (end 139 90) (width 0.2) (layer "F.Cu") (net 1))
 (segment (start 153 104) (end 153 110.3) (width 0.2) (layer "F.Cu") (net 1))
 (segment (start 168 57.8) (end 161.38 57.8) (width 0.2) (layer "F.Cu") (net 1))
 (segment (start 144 95) (end 153 104) (width 0.2) (layer "F.Cu") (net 1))
 (via (at 175.4 55.8) (size 0.6) (drill 0.3) (layers "F.Cu" "B.Cu") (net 1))
 (via (at 162 132) (size 0.6) (drill 0.3) (layers "F.Cu" "B.Cu") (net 1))
 (via (at 139 90) (size 0.6) (drill 0.3) (layers "F.Cu" "B.Cu") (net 1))
 (via (at 168 57) (size 0.6) (drill 0.3) (layers "F.Cu" "B.Cu") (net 1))
 (via (at 161.38 57.8) (size 0.6) (drill 0.3) (layers "F.Cu" "B.Cu") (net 1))
 (via (at 144 95) (size 0.6) (drill 0.3) (layers "F.Cu" "B.Cu") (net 1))
 (segment (start 161.38 57.8) (end 161.38 60) (width 0.2) (layer "B.Cu") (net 1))
 (segment (start 168 57) (end 168 56.359999) (width 0.2) (layer "B.Cu") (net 1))
 (segment (start 167.599999 115.079999) (end 167.44 114.92) (width 0.2) (layer "B.Cu") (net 1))
 (segment (start 186.49 97.462841) (end 186.49 114.92) (width 0.2) (layer "B.Cu") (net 1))
 (segment (start 149 59.92) (end 139 69.92) (width 0.2) (layer "B.Cu") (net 1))
 (segment (start 139 69.92) (end 139 90) (width 0.2) (layer "B.Cu") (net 1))
 (segment (start 167.44 114.92) (end 148.38 114.92) (width 0.2) (layer "B.Cu") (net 1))
 (segment (start 162.399998 132.399998) (end 162.399998 134.605684) (width 0.2) (layer "B.Cu") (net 1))
 (segment (start 139.600001 95.647158) (end 143.352842 95.647158) (width 0.2) (layer "B.Cu") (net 1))
 (segment (start 175.422 55.778) (end 175.4 55.8) (width 0.2) (layer "B.Cu") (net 1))
 (segment (start 177.835 55.778) (end 175.422 55.778) (width 0.2) (layer "B.Cu") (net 1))
 (segment (start 162 132) (end 162.399998 132.399998) (width 0.2) (layer "B.Cu") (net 1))
 (segment (start 190.399999 94.352842) (end 189.599999 94.352842) (width 0.2) (layer "B.Cu") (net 1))
 (segment (start 161.38 60) (end 161 60) (width 0.2) (layer "B.Cu") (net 1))
 (segment (start 143.352842 95.647158) (end 144 95) (width 0.2) (layer "B.Cu") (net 1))
 (segment (start 186.49 114.92) (end 167.44 114.92) (width 0.2) (layer "B.Cu") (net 1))
 (segment (start 189.599999 94.352842) (end 186.49 97.462841) (width 0.2) (layer "B.Cu") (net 1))
 (segment (start 168 56.359999) (end 167.600001 55.96) (width 0.2) (layer "B.Cu") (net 1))
 (segment (start 161 60) (end 160.92 59.92) (width 0.2) (layer "B.Cu") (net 1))
 (segment (start 160.92 59.92) (end 149 59.92) (width 0.2) (layer "B.Cu") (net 1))
 (segment (start 165.2 58.849) (end 165.071 58.849) (width 0.2) (layer "F.Cu") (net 7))
 (segment (start 174.649 58.849) (end 165.2 58.849) (width 0.2) (layer "F.Cu") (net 7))
 (segment (start 165.071 58.849) (end 163.92 60) (width 0.2) (layer "F.Cu") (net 7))
 (segment (start 174.8 59) (end 174.649 58.849) (width 0.2) (layer "F.Cu") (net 7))
 (via (at 174.8 59) (size 0.6) (drill 0.3) (layers "F.Cu" "B.Cu") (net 7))
 (segment (start 163.92 59.490057) (end 163.92 60) (width 0.2) (layer "B.Cu") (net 7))
 (segment (start 161.628943 57.199) (end 163.92 59.490057) (width 0.2) (layer "B.Cu") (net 7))
 (segment (start 177.835 58.165) (end 178 58) (width 0.2) (layer "B.Cu") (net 7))
 (segment (start 177.153 59) (end 174.8 59) (width 0.2) (layer "B.Cu") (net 7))
 (segment (start 177.835 58.318) (end 177.153 59) (width 0.2) (layer "B.Cu") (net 7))
 (segment (start 149.181 57.199) (end 161.628943 57.199) (width 0.2) (layer "B.Cu") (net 7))
 (segment (start 149 57.38) (end 149.181 57.199) (width 0.2) (layer "B.Cu") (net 7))
 (segment (start 195.600001 94.147158) (end 195.689915 94.147158) (width 0.2) (layer "B.Cu") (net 13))
 (segment (start 139.600001 94.147158) (end 139.600001 91.600001) (width 0.2) (layer "B.Cu") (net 4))
 (segment (start 148.118 55.96) (end 162.400001 55.96) (width 0.2) (layer "B.Cu") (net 4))
 (segment (start 139.600001 91.600001) (end 138.399 90.399) (width 0.2) (layer "B.Cu") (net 4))
 (segment (start 138.399 65.679) (end 148.118 55.96) (width 0.2) (layer "B.Cu") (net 4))
 (segment (start 138.399 90.399) (end 138.399 65.679) (width 0.2) (layer "B.Cu") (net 4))
 (segment (start 162.399998 136.105684) (end 158.620868 136.105684) (width 0.2) (layer "B.Cu") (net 12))
 (segment (start 134.400001 111.884817) (end 134.400001 95.647158) (width 0.2) (layer "B.Cu") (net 12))
 (segment (start 158.620868 136.105684) (end 134.400001 111.884817) (width 0.2) (layer "B.Cu") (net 12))
 (segment (start 172.394316 134.605684) (end 167.599998 134.605684) (width 0.2) (layer "B.Cu") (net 11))
 (segment (start 190.399999 124.600001) (end 188 127) (width 0.2) (layer "B.Cu") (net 11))
 (segment (start 190.399999 95.852842) (end 190.399999 124.600001) (width 0.2) (layer "B.Cu") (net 11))
 (segment (start 180 127) (end 172.394316 134.605684) (width 0.2) (layer "B.Cu") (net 11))
 (segment (start 188 127) (end 180 127) (width 0.2) (layer "B.Cu") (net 11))
 (segment (start 132 126) (end 140.4 134.4) (width 0.2) (layer "B.Cu") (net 3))
 (segment (start 173 52) (end 174.238 53.238) (width 0.2) (layer "B.Cu") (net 3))
 (segment (start 174.238 53.238) (end 177.835 53.238) (width 0.2) (layer "B.Cu") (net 3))
 (segment (start 167.599998 136.105684) (end 172.105684 136.105684) (width 0.2) (layer "B.Cu") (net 3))
 (segment (start 163 52) (end 135 52) (width 0.2) (layer "B.Cu") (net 3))
 (segment (start 132 91.747157) (end 132 126) (width 0.2) (layer "B.Cu") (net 3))
 (segment (start 135 52) (end 132 55) (width 0.2) (layer "B.Cu") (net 3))
 (segment (start 195.599999 119.967101) (end 195.599999 95.852842) (width 0.2) (layer "B.Cu") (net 3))
 (segment (start 140.4 134.4) (end 155.4 134.4) (width 0.2) (layer "B.Cu") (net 3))
 (segment (start 162.400001 54.46) (end 162.400001 52.599999) (width 0.2) (layer "B.Cu") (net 3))
 (segment (start 170 139) (end 172.5 136.5) (width 0.2) (layer "B.Cu") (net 3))
 (segment (start 179.400001 129.599999) (end 172.5 136.5) (width 0.2) (layer "B.Cu") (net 3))
 (segment (start 132 91.747157) (end 134.400001 94.147158) (width 0.2) (layer "B.Cu") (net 3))
 (segment (start 132 55) (end 132 91.747157) (width 0.2) (layer "B.Cu") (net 3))
 (segment (start 155.4 134.4) (end 160 139) (width 0.2) (layer "B.Cu") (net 3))
 (segment (start 160 139) (end 170 139) (width 0.2) (layer "B.Cu") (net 3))
 (segment (start 185.967101 129.599999) (end 195.599999 119.967101) (width 0.2) (layer "B.Cu") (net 3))
 (segment (start 172.105684 136.105684) (end 172.5 136.5) (width 0.2) (layer "B.Cu") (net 3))
 (segment (start 162.400001 52.599999) (end 163 52) (width 0.2) (layer "B.Cu") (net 3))
 (segment (start 163 52) (end 173 52) (width 0.2) (layer "B.Cu") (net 3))
 (segment (start 179.400001 129.599999) (end 185.967101 129.599999) (width 0.2) (layer "B.Cu") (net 3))
 (segment (start 168.400001 54.46) (end 167.600001 54.46) (width 0.2) (layer "B.Cu") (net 5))
 (segment (start 167.973465 54.74355) (end 167.883551 54.74355) (width 0.2) (layer "B.Cu") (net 5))
 (segment (start 176.620942 69.779) (end 170.151 63.309058) (width 0.2) (layer "B.Cu") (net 5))
 (segment (start 179.049058 69.779) (end 176.620942 69.779) (width 0.2) (layer "B.Cu") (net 5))
 (segment (start 187.970058 60.858) (end 179.049058 69.779) (width 0.2) (layer "B.Cu") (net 5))
 (segment (start 170.151 56.210999) (end 168.400001 54.46) (width 0.2) (layer "B.Cu") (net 5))
 (segment (start 170.151 63.309058) (end 170.151 56.210999) (width 0.2) (layer "B.Cu") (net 5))
 (segment (start 194 60.858) (end 187.970058 60.858) (width 0.2) (layer "B.Cu") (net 5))
 (segment (start 181.793794 70.18) (end 175.437919 70.18) (width 0.2) (layer "B.Cu") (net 8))
 (segment (start 166.17645 60.28355) (end 164 62.46) (width 0.2) (layer "B.Cu") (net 8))
 (segment (start 175.437919 70.18) (end 166.46 61.202081) (width 0.2) (layer "B.Cu") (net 8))
 (segment (start 186.035794 65.938) (end 181.793794 70.18) (width 0.2) (layer "B.Cu") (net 8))
 (segment (start 194 65.938) (end 186.035794 65.938) (width 0.2) (layer "B.Cu") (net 8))
 (segment (start 164 62.46) (end 149 62.46) (width 0.2) (layer "B.Cu") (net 8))
 (segment (start 166.46 61.202081) (end 166.46 60) (width 0.2) (layer "B.Cu") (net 8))
 (segment (start 169 60) (end 164.27 64.73) (width 0.2) (layer "F.Cu") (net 9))
 (via (at 164.27 64.73) (size 0.6) (drill 0.3) (layers "F.Cu" "B.Cu") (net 9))
 (segment (start 194 63.398) (end 195.676 65.074) (width 0.2) (layer "B.Cu") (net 9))
 (segment (start 164 65) (end 149 65) (width 0.2) (layer "B.Cu") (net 9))
 (segment (start 195.676 65.074) (end 195.676 69.317058) (width 0.2) (layer "B.Cu") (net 9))
 (segment (start 195.676 69.317058) (end 193.944058 71.049) (width 0.2) (layer "B.Cu") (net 9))
 (segment (start 193.944058 71.049) (end 170.589 71.049) (width 0.2) (layer "B.Cu") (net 9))
 (segment (start 164.27 64.73) (end 164 65) (width 0.2) (layer "B.Cu") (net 9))
 (segment (start 170.589 71.049) (end 164.27 64.73) (width 0.2) (layer "B.Cu") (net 9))
 (segment (start 151 109) (end 150.49 109) (width 0.2) (layer "F.Cu") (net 2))
 (segment (start 150.49 109) (end 142.03 117.46) (width 0.2) (layer "F.Cu") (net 2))
 (via (at 151 109) (size 0.6) (drill 0.3) (layers "F.Cu" "B.Cu") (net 2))
 (segment (start 196.879 56.117) (end 196.879 78.538043) (width 0.2) (layer "B.Cu") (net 2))
 (segment (start 194 53.238) (end 196.879 56.117) (width 0.2) (layer "B.Cu") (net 2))
 (segment (start 196.879 78.538043) (end 166.417043 109) (width 0.2) (layer "B.Cu") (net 2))
 (segment (start 166.417043 109) (end 151 109) (width 0.2) (layer "B.Cu") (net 2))
 (segment (start 161 104) (end 161.09 104.09) (width 0.2) (layer "F.Cu") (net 10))
 (segment (start 161.09 104.09) (end 161.09 117.46) (width 0.2) (layer "F.Cu") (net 10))
 (segment (start 161 103) (end 161 104) (width 0.2) (layer "F.Cu") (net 10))
 (via (at 161 103) (size 0.6) (drill 0.3) (layers "F.Cu" "B.Cu") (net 10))
 (segment (start 196.478 58.256) (end 196.478 78.371943) (width 0.2) (layer "B.Cu") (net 10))
 (segment (start 171.849943 103) (end 161 103) (width 0.2) (layer "B.Cu") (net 10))
 (segment (start 194 55.778) (end 196.478 58.256) (width 0.2) (layer "B.Cu") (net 10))
 (segment (start 196.478 78.371943) (end 171.849943 103) (width 0.2) (layer "B.Cu") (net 10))
 (segment (start 180.14 94.86) (end 180.14 117.46) (width 0.2) (layer "F.Cu") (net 6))
 (segment (start 181 93) (end 181 94) (width 0.2) (layer "F.Cu") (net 6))
 (segment (start 181 94) (end 180.14 94.86) (width 0.2) (layer "F.Cu") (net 6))
 (via (at 181 93) (size 0.6) (drill 0.3) (layers "F.Cu" "B.Cu") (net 6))
 (segment (start 194 58.318) (end 196.077 60.395) (width 0.2) (layer "B.Cu") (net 6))
 (segment (start 196.077 60.395) (end 196.077 77.923) (width 0.2) (layer "B.Cu") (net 6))
 (segment (start 196.077 77.923) (end 181 93) (width 0.2) (layer "B.Cu") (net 6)))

